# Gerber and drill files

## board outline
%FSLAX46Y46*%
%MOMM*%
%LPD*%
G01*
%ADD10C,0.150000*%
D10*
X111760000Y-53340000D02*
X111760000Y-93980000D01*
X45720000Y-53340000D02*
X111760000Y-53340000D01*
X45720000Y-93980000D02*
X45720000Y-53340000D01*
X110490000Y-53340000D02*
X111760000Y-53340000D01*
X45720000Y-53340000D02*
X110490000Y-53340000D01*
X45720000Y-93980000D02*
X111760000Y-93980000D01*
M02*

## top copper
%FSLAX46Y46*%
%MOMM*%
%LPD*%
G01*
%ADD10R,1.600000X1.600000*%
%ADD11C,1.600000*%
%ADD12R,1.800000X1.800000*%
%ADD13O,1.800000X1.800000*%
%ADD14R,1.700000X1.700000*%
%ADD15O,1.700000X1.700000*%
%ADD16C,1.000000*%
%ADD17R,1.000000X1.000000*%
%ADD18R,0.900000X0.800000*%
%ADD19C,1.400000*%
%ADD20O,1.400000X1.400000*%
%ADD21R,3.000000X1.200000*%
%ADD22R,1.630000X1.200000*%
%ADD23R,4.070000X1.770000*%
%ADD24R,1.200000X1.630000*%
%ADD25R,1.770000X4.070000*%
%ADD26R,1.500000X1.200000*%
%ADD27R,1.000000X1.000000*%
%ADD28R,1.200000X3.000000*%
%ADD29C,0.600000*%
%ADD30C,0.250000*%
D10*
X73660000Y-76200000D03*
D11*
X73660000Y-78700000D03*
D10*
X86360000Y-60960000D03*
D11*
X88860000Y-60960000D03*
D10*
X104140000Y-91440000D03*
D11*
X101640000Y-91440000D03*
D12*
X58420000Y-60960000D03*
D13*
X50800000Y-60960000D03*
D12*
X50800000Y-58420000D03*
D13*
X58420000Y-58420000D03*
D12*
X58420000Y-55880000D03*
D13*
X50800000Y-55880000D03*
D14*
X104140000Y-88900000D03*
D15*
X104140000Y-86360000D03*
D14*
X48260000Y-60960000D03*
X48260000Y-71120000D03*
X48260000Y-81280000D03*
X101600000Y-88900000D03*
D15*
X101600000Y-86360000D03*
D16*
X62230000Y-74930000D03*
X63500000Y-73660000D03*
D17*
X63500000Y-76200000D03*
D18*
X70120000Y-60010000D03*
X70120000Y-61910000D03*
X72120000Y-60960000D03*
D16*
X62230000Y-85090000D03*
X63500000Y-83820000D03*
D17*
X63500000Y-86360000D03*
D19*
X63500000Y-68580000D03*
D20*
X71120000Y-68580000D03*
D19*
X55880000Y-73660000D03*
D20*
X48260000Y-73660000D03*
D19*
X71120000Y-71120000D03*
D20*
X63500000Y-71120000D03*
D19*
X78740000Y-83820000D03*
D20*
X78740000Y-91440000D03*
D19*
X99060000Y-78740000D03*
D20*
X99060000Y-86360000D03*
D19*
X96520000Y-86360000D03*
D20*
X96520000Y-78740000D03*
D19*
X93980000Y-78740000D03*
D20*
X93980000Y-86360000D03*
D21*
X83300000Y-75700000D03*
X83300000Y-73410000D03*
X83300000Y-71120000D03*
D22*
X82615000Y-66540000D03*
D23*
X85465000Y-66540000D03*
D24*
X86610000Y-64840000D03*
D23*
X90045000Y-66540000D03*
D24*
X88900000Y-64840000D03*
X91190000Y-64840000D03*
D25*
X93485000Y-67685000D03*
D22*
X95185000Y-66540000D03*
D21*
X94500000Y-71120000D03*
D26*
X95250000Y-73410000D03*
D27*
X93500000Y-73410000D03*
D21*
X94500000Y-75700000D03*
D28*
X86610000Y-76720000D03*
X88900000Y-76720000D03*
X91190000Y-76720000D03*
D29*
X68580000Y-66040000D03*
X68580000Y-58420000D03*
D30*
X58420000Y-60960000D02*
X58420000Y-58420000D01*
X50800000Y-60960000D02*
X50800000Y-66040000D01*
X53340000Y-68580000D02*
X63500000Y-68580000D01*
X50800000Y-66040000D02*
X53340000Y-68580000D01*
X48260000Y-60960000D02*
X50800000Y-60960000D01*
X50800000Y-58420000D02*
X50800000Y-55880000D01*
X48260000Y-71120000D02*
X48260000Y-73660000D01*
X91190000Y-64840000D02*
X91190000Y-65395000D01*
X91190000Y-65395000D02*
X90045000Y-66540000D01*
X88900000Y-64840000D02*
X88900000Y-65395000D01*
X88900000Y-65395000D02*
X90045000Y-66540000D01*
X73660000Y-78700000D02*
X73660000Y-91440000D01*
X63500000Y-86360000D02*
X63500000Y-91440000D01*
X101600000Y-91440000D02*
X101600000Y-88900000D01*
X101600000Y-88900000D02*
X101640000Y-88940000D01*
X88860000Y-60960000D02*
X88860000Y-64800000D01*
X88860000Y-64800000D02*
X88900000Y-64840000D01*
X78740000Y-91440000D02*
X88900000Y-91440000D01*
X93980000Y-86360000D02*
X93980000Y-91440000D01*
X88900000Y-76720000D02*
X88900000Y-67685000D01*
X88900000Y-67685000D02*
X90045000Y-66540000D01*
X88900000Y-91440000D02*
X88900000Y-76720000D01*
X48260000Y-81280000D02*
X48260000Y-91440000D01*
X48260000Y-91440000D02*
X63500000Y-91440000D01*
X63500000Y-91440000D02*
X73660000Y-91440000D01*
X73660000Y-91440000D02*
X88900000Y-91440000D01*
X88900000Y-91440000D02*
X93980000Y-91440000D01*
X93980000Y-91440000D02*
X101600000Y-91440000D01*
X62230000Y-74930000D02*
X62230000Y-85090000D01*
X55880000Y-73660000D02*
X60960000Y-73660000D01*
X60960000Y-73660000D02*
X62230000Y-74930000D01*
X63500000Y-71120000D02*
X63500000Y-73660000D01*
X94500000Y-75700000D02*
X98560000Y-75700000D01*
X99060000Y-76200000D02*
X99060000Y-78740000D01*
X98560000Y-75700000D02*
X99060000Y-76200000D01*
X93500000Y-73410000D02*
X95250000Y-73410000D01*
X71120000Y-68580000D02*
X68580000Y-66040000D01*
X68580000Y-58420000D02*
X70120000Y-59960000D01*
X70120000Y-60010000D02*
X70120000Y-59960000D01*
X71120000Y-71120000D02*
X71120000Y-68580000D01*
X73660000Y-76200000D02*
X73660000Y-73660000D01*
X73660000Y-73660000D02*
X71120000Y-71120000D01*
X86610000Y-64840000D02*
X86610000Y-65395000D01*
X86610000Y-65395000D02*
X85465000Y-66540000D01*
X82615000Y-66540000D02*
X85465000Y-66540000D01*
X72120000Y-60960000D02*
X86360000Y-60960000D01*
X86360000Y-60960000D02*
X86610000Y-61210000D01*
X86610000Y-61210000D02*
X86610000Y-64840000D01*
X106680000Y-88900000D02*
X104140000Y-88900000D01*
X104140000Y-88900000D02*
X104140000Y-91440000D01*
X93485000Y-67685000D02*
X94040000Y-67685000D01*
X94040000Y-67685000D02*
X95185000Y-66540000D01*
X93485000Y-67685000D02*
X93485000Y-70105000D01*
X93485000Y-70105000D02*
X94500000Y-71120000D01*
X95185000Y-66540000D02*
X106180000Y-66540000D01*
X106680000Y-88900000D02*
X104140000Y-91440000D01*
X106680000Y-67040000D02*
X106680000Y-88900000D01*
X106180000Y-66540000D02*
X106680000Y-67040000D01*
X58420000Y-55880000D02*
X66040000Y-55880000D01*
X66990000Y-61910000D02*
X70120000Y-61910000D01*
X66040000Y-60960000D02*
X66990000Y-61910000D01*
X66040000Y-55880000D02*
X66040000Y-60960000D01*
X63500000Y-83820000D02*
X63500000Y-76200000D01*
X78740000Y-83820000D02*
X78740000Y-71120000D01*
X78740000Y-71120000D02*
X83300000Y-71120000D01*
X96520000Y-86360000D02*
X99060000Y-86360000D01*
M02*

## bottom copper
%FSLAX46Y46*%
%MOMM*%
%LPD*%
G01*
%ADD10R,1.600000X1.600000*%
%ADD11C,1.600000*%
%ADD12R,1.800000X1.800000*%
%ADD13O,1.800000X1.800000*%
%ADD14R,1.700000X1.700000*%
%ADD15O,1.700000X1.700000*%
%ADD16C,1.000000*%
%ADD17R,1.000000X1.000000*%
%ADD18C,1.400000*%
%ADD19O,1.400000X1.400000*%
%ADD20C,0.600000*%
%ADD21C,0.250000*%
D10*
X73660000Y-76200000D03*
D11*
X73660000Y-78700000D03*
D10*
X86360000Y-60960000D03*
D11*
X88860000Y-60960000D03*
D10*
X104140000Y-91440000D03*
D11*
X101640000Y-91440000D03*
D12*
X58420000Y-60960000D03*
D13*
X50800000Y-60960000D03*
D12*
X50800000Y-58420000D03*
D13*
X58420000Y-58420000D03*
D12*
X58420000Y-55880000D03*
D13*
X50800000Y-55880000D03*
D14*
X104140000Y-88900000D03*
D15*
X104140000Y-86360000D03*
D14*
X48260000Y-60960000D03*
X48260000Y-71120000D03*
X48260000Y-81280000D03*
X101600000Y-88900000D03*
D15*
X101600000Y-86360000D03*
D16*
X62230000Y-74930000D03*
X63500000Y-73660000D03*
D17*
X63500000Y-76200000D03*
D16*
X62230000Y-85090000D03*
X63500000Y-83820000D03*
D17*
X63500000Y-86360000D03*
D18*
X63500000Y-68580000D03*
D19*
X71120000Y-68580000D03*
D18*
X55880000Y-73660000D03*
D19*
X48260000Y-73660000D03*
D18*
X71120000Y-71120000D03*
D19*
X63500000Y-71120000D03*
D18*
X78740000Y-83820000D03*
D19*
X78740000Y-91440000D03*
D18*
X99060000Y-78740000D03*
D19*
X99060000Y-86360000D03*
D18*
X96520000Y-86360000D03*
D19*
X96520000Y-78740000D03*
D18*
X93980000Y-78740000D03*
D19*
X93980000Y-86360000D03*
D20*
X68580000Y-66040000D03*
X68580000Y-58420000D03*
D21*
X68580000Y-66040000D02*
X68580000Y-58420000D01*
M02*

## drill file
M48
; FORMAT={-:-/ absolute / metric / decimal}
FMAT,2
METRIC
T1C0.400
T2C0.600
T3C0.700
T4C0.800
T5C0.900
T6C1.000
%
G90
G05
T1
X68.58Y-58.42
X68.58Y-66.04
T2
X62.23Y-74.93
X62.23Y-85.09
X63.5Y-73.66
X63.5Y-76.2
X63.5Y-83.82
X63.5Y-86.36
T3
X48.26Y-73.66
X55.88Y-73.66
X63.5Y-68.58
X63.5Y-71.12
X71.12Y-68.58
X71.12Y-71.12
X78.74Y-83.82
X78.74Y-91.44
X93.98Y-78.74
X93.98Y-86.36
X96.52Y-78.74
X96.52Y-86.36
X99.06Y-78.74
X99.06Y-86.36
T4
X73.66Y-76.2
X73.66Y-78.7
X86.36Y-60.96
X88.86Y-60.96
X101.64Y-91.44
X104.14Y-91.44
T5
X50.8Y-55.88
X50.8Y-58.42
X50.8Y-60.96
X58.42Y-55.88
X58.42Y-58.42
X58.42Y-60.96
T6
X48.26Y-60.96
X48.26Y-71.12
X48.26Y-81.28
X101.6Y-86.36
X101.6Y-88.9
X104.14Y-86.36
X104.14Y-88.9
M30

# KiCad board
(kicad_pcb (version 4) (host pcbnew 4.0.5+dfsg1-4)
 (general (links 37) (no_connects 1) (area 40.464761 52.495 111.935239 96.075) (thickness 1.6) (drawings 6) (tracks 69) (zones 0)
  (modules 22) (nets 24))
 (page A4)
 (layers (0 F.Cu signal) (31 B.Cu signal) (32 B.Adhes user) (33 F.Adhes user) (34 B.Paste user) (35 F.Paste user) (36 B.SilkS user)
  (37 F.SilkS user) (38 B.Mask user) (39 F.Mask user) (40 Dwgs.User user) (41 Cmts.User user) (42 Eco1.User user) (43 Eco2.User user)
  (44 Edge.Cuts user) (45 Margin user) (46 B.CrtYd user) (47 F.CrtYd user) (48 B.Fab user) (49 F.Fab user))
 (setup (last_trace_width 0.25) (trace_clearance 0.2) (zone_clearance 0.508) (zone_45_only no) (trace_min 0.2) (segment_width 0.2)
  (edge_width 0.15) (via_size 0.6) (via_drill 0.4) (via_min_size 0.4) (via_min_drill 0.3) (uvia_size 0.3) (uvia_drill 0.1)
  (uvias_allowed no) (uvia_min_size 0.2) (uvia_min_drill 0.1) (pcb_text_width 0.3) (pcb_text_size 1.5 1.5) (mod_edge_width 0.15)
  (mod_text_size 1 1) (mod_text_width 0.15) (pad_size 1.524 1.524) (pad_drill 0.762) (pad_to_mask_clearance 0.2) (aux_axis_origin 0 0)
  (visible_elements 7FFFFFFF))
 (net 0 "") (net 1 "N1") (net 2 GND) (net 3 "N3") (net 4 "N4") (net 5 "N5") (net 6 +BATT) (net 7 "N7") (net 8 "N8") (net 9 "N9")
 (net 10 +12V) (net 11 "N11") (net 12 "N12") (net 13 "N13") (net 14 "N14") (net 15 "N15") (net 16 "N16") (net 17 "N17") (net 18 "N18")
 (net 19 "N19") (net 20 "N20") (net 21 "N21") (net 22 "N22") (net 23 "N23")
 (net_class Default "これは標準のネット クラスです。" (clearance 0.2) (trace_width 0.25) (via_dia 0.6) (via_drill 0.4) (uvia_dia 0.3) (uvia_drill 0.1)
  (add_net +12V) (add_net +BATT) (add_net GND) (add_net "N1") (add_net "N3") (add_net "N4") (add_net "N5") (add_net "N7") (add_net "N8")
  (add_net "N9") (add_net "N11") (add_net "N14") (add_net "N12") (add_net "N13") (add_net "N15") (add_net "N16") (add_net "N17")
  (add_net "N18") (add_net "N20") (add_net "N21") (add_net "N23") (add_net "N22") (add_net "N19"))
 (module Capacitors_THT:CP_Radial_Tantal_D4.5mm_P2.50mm (layer F.Cu) (at 73.66 76.2 270)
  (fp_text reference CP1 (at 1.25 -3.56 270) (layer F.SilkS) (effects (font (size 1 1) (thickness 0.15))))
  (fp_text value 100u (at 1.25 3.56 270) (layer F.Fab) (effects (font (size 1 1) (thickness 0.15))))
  (pad 1 thru_hole rect (at 0 0 270) (size 1.6 1.6) (drill 0.8) (layers *.Cu *.Mask) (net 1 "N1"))
  (pad 2 thru_hole circle (at 2.5 0 270) (size 1.6 1.6) (drill 0.8) (layers *.Cu *.Mask) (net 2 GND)))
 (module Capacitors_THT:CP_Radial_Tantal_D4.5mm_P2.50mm (layer F.Cu) (at 86.36 60.96)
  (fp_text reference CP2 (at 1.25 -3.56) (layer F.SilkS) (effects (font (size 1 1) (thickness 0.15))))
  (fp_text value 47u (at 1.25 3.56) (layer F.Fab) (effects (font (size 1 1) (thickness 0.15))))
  (pad 1 thru_hole rect (at 0 0) (size 1.6 1.6) (drill 0.8) (layers *.Cu *.Mask) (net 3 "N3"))
  (pad 2 thru_hole circle (at 2.5 0) (size 1.6 1.6) (drill 0.8) (layers *.Cu *.Mask) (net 2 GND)))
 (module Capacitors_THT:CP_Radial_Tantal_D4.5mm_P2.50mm (layer F.Cu) (at 104.14 91.44 180)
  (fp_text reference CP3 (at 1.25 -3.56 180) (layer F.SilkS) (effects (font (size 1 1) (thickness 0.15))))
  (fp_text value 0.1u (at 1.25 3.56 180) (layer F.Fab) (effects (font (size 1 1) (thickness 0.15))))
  (pad 1 thru_hole rect (at 0 0 180) (size 1.6 1.6) (drill 0.8) (layers *.Cu *.Mask) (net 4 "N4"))
  (pad 2 thru_hole circle (at 2.5 0 180) (size 1.6 1.6) (drill 0.8) (layers *.Cu *.Mask) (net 2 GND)))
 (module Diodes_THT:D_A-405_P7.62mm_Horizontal (layer F.Cu) (at 58.42 60.96 180)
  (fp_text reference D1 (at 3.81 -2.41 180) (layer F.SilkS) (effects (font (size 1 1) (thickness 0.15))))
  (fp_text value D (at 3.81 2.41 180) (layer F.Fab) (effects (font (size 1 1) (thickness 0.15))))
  (pad 1 thru_hole rect (at 0 0 180) (size 1.8 1.8) (drill 0.9) (layers *.Cu *.Mask) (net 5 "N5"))
  (pad 2 thru_hole oval (at 7.62 0 180) (size 1.8 1.8) (drill 0.9) (layers *.Cu *.Mask) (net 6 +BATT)))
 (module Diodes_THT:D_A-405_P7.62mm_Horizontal (layer F.Cu) (at 50.8 58.42)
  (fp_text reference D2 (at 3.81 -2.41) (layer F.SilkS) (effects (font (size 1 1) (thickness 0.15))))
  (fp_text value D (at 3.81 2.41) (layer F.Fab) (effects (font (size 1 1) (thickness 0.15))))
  (pad 1 thru_hole rect (at 0 0) (size 1.8 1.8) (drill 0.9) (layers *.Cu *.Mask) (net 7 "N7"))
  (pad 2 thru_hole oval (at 7.62 0) (size 1.8 1.8) (drill 0.9) (layers *.Cu *.Mask) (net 5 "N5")))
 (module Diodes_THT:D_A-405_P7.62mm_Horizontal (layer F.Cu) (at 58.42 55.88 180)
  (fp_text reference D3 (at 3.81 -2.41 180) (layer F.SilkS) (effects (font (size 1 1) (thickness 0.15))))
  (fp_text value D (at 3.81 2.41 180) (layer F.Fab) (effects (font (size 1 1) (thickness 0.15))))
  (pad 1 thru_hole rect (at 0 0 180) (size 1.8 1.8) (drill 0.9) (layers *.Cu *.Mask) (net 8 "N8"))
  (pad 2 thru_hole oval (at 7.62 0 180) (size 1.8 1.8) (drill 0.9) (layers *.Cu *.Mask) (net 7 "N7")))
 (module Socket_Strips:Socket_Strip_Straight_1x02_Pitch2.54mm (layer F.Cu) (at 104.14 88.9 180)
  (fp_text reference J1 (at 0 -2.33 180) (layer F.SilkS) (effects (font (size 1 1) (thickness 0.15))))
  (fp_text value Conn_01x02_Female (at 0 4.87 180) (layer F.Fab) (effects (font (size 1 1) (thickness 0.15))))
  (pad 1 thru_hole rect (at 0 0 180) (size 1.7 1.7) (drill 1) (layers *.Cu *.Mask) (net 4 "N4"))
  (pad 2 thru_hole oval (at 0 2.54 180) (size 1.7 1.7) (drill 1) (layers *.Cu *.Mask) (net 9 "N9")))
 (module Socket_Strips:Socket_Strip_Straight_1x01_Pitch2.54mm (layer F.Cu) (at 48.26 60.96)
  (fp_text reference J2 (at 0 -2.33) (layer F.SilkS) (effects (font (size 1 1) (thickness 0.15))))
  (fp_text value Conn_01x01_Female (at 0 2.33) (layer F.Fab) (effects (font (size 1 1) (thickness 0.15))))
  (pad 1 thru_hole rect (at 0 0) (size 1.7 1.7) (drill 1) (layers *.Cu *.Mask) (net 6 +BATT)))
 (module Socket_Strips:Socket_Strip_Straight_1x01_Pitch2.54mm (layer F.Cu) (at 48.26 71.12)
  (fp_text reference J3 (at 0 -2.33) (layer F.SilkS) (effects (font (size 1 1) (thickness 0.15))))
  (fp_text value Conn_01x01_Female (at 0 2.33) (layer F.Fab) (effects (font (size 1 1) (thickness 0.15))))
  (pad 1 thru_hole rect (at 0 0) (size 1.7 1.7) (drill 1) (layers *.Cu *.Mask) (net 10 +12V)))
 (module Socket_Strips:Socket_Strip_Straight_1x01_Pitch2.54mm (layer F.Cu) (at 48.26 81.28)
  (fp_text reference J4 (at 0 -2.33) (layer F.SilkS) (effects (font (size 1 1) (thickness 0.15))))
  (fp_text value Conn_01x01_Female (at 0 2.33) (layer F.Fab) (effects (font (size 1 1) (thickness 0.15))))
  (pad 1 thru_hole rect (at 0 0) (size 1.7 1.7) (drill 1) (layers *.Cu *.Mask) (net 2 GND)))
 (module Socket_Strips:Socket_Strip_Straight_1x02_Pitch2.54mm (layer F.Cu) (at 101.6 88.9 180)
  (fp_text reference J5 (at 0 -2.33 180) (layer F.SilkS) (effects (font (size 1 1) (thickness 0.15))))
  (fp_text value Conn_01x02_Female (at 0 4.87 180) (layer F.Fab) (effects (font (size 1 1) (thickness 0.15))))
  (pad 1 thru_hole rect (at 0 0 180) (size 1.7 1.7) (drill 1) (layers *.Cu *.Mask) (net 2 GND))
  (pad 2 thru_hole oval (at 0 2.54 180) (size 1.7 1.7) (drill 1) (layers *.Cu *.Mask) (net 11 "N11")))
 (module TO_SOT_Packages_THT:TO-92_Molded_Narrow (layer F.Cu) (at 63.5 76.2 90)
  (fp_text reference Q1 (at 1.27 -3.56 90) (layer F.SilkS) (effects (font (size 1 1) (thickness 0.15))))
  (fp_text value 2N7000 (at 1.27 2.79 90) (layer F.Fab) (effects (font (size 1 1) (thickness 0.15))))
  (pad 2 thru_hole circle (at 1.27 -1.27 180) (size 1 1) (drill 0.6) (layers *.Cu *.Mask) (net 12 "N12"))
  (pad 3 thru_hole circle (at 2.54 0 180) (size 1 1) (drill 0.6) (layers *.Cu *.Mask) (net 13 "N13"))
  (pad 1 thru_hole rect (at 0 0 180) (size 1 1) (drill 0.6) (layers *.Cu *.Mask) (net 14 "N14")))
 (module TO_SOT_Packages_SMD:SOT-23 (layer F.Cu) (at 71.12 60.96)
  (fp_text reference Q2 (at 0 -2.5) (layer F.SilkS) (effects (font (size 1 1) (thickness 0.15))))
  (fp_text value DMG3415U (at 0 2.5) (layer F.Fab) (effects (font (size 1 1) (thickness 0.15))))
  (pad 1 smd rect (at -1 -0.95) (size 0.9 0.8) (layers F.Cu F.Paste F.Mask) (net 1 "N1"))
  (pad 2 smd rect (at -1 0.95) (size 0.9 0.8) (layers F.Cu F.Paste F.Mask) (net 8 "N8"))
  (pad 3 smd rect (at 1 0) (size 0.9 0.8) (layers F.Cu F.Paste F.Mask) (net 3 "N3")))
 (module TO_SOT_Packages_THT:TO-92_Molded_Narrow (layer F.Cu) (at 63.5 86.36 90)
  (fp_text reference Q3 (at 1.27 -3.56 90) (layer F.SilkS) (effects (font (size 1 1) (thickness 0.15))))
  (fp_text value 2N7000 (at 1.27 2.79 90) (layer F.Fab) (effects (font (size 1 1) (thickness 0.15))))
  (pad 2 thru_hole circle (at 1.27 -1.27 180) (size 1 1) (drill 0.6) (layers *.Cu *.Mask) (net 12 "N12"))
  (pad 3 thru_hole circle (at 2.54 0 180) (size 1 1) (drill 0.6) (layers *.Cu *.Mask) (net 14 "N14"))
  (pad 1 thru_hole rect (at 0 0 180) (size 1 1) (drill 0.6) (layers *.Cu *.Mask) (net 2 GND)))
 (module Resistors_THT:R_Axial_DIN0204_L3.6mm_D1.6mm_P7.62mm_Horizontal (layer F.Cu) (at 63.5 68.58)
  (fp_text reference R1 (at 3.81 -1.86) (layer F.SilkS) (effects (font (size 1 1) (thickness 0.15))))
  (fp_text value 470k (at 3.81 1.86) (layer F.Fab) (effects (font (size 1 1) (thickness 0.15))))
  (pad 1 thru_hole circle (at 0 0) (size 1.4 1.4) (drill 0.7) (layers *.Cu *.Mask) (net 6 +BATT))
  (pad 2 thru_hole oval (at 7.62 0) (size 1.4 1.4) (drill 0.7) (layers *.Cu *.Mask) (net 1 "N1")))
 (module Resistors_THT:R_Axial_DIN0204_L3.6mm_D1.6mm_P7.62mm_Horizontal (layer F.Cu) (at 55.88 73.66 180)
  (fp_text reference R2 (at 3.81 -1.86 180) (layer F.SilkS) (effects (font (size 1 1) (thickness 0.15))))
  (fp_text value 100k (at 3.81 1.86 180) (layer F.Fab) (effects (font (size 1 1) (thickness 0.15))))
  (pad 1 thru_hole circle (at 0 0 180) (size 1.4 1.4) (drill 0.7) (layers *.Cu *.Mask) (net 12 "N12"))
  (pad 2 thru_hole oval (at 7.62 0 180) (size 1.4 1.4) (drill 0.7) (layers *.Cu *.Mask) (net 10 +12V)))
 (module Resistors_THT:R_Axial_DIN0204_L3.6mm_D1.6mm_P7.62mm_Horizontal (layer F.Cu) (at 71.12 71.12 180)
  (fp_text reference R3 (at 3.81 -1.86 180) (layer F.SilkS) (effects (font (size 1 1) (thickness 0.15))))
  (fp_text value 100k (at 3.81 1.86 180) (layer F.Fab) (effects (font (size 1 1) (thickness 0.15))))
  (pad 1 thru_hole circle (at 0 0 180) (size 1.4 1.4) (drill 0.7) (layers *.Cu *.Mask) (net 1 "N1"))
  (pad 2 thru_hole oval (at 7.62 0 180) (size 1.4 1.4) (drill 0.7) (layers *.Cu *.Mask) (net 13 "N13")))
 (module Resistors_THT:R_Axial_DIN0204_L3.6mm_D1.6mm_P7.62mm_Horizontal (layer F.Cu) (at 78.74 83.82 270)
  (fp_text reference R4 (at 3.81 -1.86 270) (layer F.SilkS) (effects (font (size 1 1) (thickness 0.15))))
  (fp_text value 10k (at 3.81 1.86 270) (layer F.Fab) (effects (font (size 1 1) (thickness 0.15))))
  (pad 1 thru_hole circle (at 0 0 270) (size 1.4 1.4) (drill 0.7) (layers *.Cu *.Mask) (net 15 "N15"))
  (pad 2 thru_hole oval (at 7.62 0 270) (size 1.4 1.4) (drill 0.7) (layers *.Cu *.Mask) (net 2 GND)))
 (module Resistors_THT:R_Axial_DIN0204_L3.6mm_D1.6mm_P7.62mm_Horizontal (layer F.Cu) (at 99.06 78.74 270)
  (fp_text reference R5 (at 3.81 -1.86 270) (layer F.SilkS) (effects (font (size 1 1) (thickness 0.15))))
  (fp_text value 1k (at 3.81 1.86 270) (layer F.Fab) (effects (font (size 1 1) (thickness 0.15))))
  (pad 1 thru_hole circle (at 0 0 270) (size 1.4 1.4) (drill 0.7) (layers *.Cu *.Mask) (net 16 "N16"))
  (pad 2 thru_hole oval (at 7.62 0 270) (size 1.4 1.4) (drill 0.7) (layers *.Cu *.Mask) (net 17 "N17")))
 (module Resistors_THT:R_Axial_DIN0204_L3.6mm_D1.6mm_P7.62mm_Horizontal (layer F.Cu) (at 96.52 86.36 90)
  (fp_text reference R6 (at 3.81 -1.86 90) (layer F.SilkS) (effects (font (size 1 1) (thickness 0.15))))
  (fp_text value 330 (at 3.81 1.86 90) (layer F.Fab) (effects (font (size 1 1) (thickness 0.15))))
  (pad 1 thru_hole circle (at 0 0 90) (size 1.4 1.4) (drill 0.7) (layers *.Cu *.Mask) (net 17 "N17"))
  (pad 2 thru_hole oval (at 7.62 0 90) (size 1.4 1.4) (drill 0.7) (layers *.Cu *.Mask) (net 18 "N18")))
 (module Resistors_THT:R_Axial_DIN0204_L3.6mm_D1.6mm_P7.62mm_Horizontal (layer F.Cu) (at 93.98 78.74 270)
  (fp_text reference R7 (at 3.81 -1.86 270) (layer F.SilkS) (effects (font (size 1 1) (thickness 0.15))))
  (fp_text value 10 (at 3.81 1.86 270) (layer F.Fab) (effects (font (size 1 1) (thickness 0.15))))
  (pad 1 thru_hole circle (at 0 0 270) (size 1.4 1.4) (drill 0.7) (layers *.Cu *.Mask) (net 18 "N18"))
  (pad 2 thru_hole oval (at 7.62 0 270) (size 1.4 1.4) (drill 0.7) (layers *.Cu *.Mask) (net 2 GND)))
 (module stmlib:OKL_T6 (layer F.Cu) (at 88.9 71.12)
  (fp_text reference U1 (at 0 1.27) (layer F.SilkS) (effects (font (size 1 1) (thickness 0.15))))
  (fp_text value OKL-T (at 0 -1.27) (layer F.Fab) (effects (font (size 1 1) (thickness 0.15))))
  (pad 9 smd rect (at -5.6 4.58) (size 3 1.2) (layers F.Cu F.Paste F.Mask) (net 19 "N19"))
  (pad 10 smd rect (at -5.6 2.29) (size 3 1.2) (layers F.Cu F.Paste F.Mask) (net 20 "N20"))
  (pad 1 smd rect (at -5.6 0) (size 3 1.2) (layers F.Cu F.Paste F.Mask) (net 15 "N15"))
  (pad 2 smd rect (at -6.285 -4.58) (size 1.63 1.2) (layers F.Cu F.Paste F.Mask) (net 3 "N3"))
  (pad 2 smd rect (at -3.435 -4.58) (size 4.07 1.77) (layers F.Cu F.Paste F.Mask) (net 3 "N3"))
  (pad 2 smd rect (at -2.29 -6.28) (size 1.2 1.63) (layers F.Cu F.Paste F.Mask) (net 3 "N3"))
  (pad 3 smd rect (at 1.145 -4.58) (size 4.07 1.77) (layers F.Cu F.Paste F.Mask) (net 2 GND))
  (pad 3 smd rect (at 0 -6.28) (size 1.2 1.63) (layers F.Cu F.Paste F.Mask) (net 2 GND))
  (pad 3 smd rect (at 2.29 -6.28) (size 1.2 1.63) (layers F.Cu F.Paste F.Mask) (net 2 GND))
  (pad 4 smd rect (at 4.585 -3.435) (size 1.77 4.07) (layers F.Cu F.Paste F.Mask) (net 4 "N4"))
  (pad 4 smd rect (at 6.285 -4.58) (size 1.63 1.2) (layers F.Cu F.Paste F.Mask) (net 4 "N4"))
  (pad 5 smd rect (at 5.6 0) (size 3 1.2) (layers F.Cu F.Paste F.Mask) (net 4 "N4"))
  (pad 11 smd rect (at 6.35 2.29) (size 1.5 1.2) (layers F.Cu F.Paste F.Mask) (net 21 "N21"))
  (pad 11 smd rect (at 4.6 2.29) (size 1 1) (layers F.Cu F.Paste F.Mask) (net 21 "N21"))
  (pad 6 smd rect (at 5.6 4.58) (size 3 1.2) (layers F.Cu F.Paste F.Mask) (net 16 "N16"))
  (pad 8 smd rect (at -2.29 5.6) (size 1.2 3) (layers F.Cu F.Paste F.Mask) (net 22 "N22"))
  (pad 7 smd rect (at 0 5.6) (size 1.2 3) (layers F.Cu F.Paste F.Mask) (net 2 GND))
  (pad 12 smd rect (at 2.29 5.6) (size 1.2 3) (layers F.Cu F.Paste F.Mask) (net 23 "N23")))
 (gr_line (start 111.76 53.34) (end 111.76 93.98) (angle 90) (layer Edge.Cuts) (width 0.15))
 (gr_line (start 45.72 53.34) (end 111.76 53.34) (angle 90) (layer Edge.Cuts) (width 0.15))
 (gr_line (start 45.72 93.98) (end 45.72 53.34) (angle 90) (layer Edge.Cuts) (width 0.15))
 (gr_line (start 110.49 53.34) (end 111.76 53.34) (angle 90) (layer Edge.Cuts) (width 0.15))
 (gr_line (start 45.72 53.34) (end 110.49 53.34) (angle 90) (layer Edge.Cuts) (width 0.15))
 (gr_line (start 45.72 93.98) (end 111.76 93.98) (angle 90) (layer Edge.Cuts) (width 0.15))
 (segment (start 58.42 60.96) (end 58.42 58.42) (width 0.25) (layer F.Cu) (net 5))
 (segment (start 50.8 60.96) (end 50.8 66.04) (width 0.25) (layer F.Cu) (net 6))
 (segment (start 53.34 68.58) (end 63.5 68.58) (width 0.25) (layer F.Cu) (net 6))
 (segment (start 50.8 66.04) (end 53.34 68.58) (width 0.25) (layer F.Cu) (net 6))
 (segment (start 48.26 60.96) (end 50.8 60.96) (width 0.25) (layer F.Cu) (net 6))
 (segment (start 50.8 58.42) (end 50.8 55.88) (width 0.25) (layer F.Cu) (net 7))
 (segment (start 48.26 71.12) (end 48.26 73.66) (width 0.25) (layer F.Cu) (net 10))
 (segment (start 91.19 64.84) (end 91.19 65.395) (width 0.25) (layer F.Cu) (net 2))
 (segment (start 91.19 65.395) (end 90.045 66.54) (width 0.25) (layer F.Cu) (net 2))
 (segment (start 88.9 64.84) (end 88.9 65.395) (width 0.25) (layer F.Cu) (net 2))
 (segment (start 88.9 65.395) (end 90.045 66.54) (width 0.25) (layer F.Cu) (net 2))
 (segment (start 73.66 78.7) (end 73.66 91.44) (width 0.25) (layer F.Cu) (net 2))
 (segment (start 63.5 86.36) (end 63.5 91.44) (width 0.25) (layer F.Cu) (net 2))
 (segment (start 101.6 91.44) (end 101.6 88.9) (width 0.25) (layer F.Cu) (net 2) (status 800000))
 (segment (start 101.6 88.9) (end 101.64 88.94) (width 0.25) (layer F.Cu) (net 2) (status 400000))
 (segment (start 88.86 60.96) (end 88.86 64.8) (width 0.25) (layer F.Cu) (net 2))
 (segment (start 88.86 64.8) (end 88.9 64.84) (width 0.25) (layer F.Cu) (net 2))
 (segment (start 78.74 91.44) (end 88.9 91.44) (width 0.25) (layer F.Cu) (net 2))
 (segment (start 93.98 86.36) (end 93.98 91.44) (width 0.25) (layer F.Cu) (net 2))
 (segment (start 88.9 76.72) (end 88.9 67.685) (width 0.25) (layer F.Cu) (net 2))
 (segment (start 88.9 67.685) (end 90.045 66.54) (width 0.25) (layer F.Cu) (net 2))
 (segment (start 88.9 91.44) (end 88.9 76.72) (width 0.25) (layer F.Cu) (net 2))
 (segment (start 48.26 81.28) (end 48.26 91.44) (width 0.25) (layer F.Cu) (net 2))
 (segment (start 48.26 91.44) (end 63.5 91.44) (width 0.25) (layer F.Cu) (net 2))
 (segment (start 63.5 91.44) (end 73.66 91.44) (width 0.25) (layer F.Cu) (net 2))
 (segment (start 73.66 91.44) (end 88.9 91.44) (width 0.25) (layer F.Cu) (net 2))
 (segment (start 88.9 91.44) (end 93.98 91.44) (width 0.25) (layer F.Cu) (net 2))
 (segment (start 93.98 91.44) (end 101.6 91.44) (width 0.25) (layer F.Cu) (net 2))
 (segment (start 62.23 74.93) (end 62.23 85.09) (width 0.25) (layer F.Cu) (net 12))
 (segment (start 55.88 73.66) (end 60.96 73.66) (width 0.25) (layer F.Cu) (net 12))
 (segment (start 60.96 73.66) (end 62.23 74.93) (width 0.25) (layer F.Cu) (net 12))
 (segment (start 63.5 71.12) (end 63.5 73.66) (width 0.25) (layer F.Cu) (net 13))
 (segment (start 94.5 75.7) (end 98.56 75.7) (width 0.25) (layer F.Cu) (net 16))
 (segment (start 99.06 76.2) (end 99.06 78.74) (width 0.25) (layer F.Cu) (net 16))
 (segment (start 98.56 75.7) (end 99.06 76.2) (width 0.25) (layer F.Cu) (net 16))
 (segment (start 93.5 73.41) (end 95.25 73.41) (width 0.25) (layer F.Cu) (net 21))
 (via (at 68.58 66.04) (size 0.6) (drill 0.4) (layers F.Cu B.Cu) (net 1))
 (segment (start 71.12 68.58) (end 68.58 66.04) (width 0.25) (layer F.Cu) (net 1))
 (segment (start 68.58 58.42) (end 70.12 59.96) (width 0.25) (layer F.Cu) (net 1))
 (via (at 68.58 58.42) (size 0.6) (drill 0.4) (layers F.Cu B.Cu) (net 1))
 (segment (start 68.58 66.04) (end 68.58 58.42) (width 0.25) (layer B.Cu) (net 1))
 (segment (start 70.12 60.01) (end 70.12 59.96) (width 0.25) (layer F.Cu) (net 1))
 (segment (start 71.12 71.12) (end 71.12 68.58) (width 0.25) (layer F.Cu) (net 1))
 (segment (start 73.66 76.2) (end 73.66 73.66) (width 0.25) (layer F.Cu) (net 1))
 (segment (start 73.66 73.66) (end 71.12 71.12) (width 0.25) (layer F.Cu) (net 1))
 (segment (start 86.61 64.84) (end 86.61 65.395) (width 0.25) (layer F.Cu) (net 3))
 (segment (start 86.61 65.395) (end 85.465 66.54) (width 0.25) (layer F.Cu) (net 3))
 (segment (start 82.615 66.54) (end 85.465 66.54) (width 0.25) (layer F.Cu) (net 3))
 (segment (start 72.12 60.96) (end 86.36 60.96) (width 0.25) (layer F.Cu) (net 3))
 (segment (start 86.36 60.96) (end 86.61 61.21) (width 0.25) (layer F.Cu) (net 3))
 (segment (start 86.61 61.21) (end 86.61 64.84) (width 0.25) (layer F.Cu) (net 3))
 (segment (start 106.68 88.9) (end 104.14 88.9) (width 0.25) (layer F.Cu) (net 4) (status 800000))
 (segment (start 104.14 88.9) (end 104.14 91.44) (width 0.25) (layer F.Cu) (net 4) (status C00000))
 (segment (start 93.485 67.685) (end 94.04 67.685) (width 0.25) (layer F.Cu) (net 4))
 (segment (start 94.04 67.685) (end 95.185 66.54) (width 0.25) (layer F.Cu) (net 4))
 (segment (start 93.485 67.685) (end 93.485 70.105) (width 0.25) (layer F.Cu) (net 4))
 (segment (start 93.485 70.105) (end 94.5 71.12) (width 0.25) (layer F.Cu) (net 4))
 (segment (start 95.185 66.54) (end 106.18 66.54) (width 0.25) (layer F.Cu) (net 4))
 (segment (start 106.68 88.9) (end 104.14 91.44) (width 0.25) (layer F.Cu) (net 4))
 (segment (start 106.68 67.04) (end 106.68 88.9) (width 0.25) (layer F.Cu) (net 4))
 (segment (start 106.18 66.54) (end 106.68 67.04) (width 0.25) (layer F.Cu) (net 4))
 (segment (start 58.42 55.88) (end 66.04 55.88) (width 0.25) (layer F.Cu) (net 8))
 (segment (start 66.99 61.91) (end 70.12 61.91) (width 0.25) (layer F.Cu) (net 8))
 (segment (start 66.04 60.96) (end 66.99 61.91) (width 0.25) (layer F.Cu) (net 8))
 (segment (start 66.04 55.88) (end 66.04 60.96) (width 0.25) (layer F.Cu) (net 8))
 (segment (start 63.5 83.82) (end 63.5 76.2) (width 0.25) (layer F.Cu) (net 14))
 (segment (start 78.74 83.82) (end 78.74 71.12) (width 0.25) (layer F.Cu) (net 15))
 (segment (start 78.74 71.12) (end 83.3 71.12) (width 0.25) (layer F.Cu) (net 15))
 (segment (start 96.52 86.36) (end 99.06 86.36) (width 0.25) (layer F.Cu) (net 17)))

